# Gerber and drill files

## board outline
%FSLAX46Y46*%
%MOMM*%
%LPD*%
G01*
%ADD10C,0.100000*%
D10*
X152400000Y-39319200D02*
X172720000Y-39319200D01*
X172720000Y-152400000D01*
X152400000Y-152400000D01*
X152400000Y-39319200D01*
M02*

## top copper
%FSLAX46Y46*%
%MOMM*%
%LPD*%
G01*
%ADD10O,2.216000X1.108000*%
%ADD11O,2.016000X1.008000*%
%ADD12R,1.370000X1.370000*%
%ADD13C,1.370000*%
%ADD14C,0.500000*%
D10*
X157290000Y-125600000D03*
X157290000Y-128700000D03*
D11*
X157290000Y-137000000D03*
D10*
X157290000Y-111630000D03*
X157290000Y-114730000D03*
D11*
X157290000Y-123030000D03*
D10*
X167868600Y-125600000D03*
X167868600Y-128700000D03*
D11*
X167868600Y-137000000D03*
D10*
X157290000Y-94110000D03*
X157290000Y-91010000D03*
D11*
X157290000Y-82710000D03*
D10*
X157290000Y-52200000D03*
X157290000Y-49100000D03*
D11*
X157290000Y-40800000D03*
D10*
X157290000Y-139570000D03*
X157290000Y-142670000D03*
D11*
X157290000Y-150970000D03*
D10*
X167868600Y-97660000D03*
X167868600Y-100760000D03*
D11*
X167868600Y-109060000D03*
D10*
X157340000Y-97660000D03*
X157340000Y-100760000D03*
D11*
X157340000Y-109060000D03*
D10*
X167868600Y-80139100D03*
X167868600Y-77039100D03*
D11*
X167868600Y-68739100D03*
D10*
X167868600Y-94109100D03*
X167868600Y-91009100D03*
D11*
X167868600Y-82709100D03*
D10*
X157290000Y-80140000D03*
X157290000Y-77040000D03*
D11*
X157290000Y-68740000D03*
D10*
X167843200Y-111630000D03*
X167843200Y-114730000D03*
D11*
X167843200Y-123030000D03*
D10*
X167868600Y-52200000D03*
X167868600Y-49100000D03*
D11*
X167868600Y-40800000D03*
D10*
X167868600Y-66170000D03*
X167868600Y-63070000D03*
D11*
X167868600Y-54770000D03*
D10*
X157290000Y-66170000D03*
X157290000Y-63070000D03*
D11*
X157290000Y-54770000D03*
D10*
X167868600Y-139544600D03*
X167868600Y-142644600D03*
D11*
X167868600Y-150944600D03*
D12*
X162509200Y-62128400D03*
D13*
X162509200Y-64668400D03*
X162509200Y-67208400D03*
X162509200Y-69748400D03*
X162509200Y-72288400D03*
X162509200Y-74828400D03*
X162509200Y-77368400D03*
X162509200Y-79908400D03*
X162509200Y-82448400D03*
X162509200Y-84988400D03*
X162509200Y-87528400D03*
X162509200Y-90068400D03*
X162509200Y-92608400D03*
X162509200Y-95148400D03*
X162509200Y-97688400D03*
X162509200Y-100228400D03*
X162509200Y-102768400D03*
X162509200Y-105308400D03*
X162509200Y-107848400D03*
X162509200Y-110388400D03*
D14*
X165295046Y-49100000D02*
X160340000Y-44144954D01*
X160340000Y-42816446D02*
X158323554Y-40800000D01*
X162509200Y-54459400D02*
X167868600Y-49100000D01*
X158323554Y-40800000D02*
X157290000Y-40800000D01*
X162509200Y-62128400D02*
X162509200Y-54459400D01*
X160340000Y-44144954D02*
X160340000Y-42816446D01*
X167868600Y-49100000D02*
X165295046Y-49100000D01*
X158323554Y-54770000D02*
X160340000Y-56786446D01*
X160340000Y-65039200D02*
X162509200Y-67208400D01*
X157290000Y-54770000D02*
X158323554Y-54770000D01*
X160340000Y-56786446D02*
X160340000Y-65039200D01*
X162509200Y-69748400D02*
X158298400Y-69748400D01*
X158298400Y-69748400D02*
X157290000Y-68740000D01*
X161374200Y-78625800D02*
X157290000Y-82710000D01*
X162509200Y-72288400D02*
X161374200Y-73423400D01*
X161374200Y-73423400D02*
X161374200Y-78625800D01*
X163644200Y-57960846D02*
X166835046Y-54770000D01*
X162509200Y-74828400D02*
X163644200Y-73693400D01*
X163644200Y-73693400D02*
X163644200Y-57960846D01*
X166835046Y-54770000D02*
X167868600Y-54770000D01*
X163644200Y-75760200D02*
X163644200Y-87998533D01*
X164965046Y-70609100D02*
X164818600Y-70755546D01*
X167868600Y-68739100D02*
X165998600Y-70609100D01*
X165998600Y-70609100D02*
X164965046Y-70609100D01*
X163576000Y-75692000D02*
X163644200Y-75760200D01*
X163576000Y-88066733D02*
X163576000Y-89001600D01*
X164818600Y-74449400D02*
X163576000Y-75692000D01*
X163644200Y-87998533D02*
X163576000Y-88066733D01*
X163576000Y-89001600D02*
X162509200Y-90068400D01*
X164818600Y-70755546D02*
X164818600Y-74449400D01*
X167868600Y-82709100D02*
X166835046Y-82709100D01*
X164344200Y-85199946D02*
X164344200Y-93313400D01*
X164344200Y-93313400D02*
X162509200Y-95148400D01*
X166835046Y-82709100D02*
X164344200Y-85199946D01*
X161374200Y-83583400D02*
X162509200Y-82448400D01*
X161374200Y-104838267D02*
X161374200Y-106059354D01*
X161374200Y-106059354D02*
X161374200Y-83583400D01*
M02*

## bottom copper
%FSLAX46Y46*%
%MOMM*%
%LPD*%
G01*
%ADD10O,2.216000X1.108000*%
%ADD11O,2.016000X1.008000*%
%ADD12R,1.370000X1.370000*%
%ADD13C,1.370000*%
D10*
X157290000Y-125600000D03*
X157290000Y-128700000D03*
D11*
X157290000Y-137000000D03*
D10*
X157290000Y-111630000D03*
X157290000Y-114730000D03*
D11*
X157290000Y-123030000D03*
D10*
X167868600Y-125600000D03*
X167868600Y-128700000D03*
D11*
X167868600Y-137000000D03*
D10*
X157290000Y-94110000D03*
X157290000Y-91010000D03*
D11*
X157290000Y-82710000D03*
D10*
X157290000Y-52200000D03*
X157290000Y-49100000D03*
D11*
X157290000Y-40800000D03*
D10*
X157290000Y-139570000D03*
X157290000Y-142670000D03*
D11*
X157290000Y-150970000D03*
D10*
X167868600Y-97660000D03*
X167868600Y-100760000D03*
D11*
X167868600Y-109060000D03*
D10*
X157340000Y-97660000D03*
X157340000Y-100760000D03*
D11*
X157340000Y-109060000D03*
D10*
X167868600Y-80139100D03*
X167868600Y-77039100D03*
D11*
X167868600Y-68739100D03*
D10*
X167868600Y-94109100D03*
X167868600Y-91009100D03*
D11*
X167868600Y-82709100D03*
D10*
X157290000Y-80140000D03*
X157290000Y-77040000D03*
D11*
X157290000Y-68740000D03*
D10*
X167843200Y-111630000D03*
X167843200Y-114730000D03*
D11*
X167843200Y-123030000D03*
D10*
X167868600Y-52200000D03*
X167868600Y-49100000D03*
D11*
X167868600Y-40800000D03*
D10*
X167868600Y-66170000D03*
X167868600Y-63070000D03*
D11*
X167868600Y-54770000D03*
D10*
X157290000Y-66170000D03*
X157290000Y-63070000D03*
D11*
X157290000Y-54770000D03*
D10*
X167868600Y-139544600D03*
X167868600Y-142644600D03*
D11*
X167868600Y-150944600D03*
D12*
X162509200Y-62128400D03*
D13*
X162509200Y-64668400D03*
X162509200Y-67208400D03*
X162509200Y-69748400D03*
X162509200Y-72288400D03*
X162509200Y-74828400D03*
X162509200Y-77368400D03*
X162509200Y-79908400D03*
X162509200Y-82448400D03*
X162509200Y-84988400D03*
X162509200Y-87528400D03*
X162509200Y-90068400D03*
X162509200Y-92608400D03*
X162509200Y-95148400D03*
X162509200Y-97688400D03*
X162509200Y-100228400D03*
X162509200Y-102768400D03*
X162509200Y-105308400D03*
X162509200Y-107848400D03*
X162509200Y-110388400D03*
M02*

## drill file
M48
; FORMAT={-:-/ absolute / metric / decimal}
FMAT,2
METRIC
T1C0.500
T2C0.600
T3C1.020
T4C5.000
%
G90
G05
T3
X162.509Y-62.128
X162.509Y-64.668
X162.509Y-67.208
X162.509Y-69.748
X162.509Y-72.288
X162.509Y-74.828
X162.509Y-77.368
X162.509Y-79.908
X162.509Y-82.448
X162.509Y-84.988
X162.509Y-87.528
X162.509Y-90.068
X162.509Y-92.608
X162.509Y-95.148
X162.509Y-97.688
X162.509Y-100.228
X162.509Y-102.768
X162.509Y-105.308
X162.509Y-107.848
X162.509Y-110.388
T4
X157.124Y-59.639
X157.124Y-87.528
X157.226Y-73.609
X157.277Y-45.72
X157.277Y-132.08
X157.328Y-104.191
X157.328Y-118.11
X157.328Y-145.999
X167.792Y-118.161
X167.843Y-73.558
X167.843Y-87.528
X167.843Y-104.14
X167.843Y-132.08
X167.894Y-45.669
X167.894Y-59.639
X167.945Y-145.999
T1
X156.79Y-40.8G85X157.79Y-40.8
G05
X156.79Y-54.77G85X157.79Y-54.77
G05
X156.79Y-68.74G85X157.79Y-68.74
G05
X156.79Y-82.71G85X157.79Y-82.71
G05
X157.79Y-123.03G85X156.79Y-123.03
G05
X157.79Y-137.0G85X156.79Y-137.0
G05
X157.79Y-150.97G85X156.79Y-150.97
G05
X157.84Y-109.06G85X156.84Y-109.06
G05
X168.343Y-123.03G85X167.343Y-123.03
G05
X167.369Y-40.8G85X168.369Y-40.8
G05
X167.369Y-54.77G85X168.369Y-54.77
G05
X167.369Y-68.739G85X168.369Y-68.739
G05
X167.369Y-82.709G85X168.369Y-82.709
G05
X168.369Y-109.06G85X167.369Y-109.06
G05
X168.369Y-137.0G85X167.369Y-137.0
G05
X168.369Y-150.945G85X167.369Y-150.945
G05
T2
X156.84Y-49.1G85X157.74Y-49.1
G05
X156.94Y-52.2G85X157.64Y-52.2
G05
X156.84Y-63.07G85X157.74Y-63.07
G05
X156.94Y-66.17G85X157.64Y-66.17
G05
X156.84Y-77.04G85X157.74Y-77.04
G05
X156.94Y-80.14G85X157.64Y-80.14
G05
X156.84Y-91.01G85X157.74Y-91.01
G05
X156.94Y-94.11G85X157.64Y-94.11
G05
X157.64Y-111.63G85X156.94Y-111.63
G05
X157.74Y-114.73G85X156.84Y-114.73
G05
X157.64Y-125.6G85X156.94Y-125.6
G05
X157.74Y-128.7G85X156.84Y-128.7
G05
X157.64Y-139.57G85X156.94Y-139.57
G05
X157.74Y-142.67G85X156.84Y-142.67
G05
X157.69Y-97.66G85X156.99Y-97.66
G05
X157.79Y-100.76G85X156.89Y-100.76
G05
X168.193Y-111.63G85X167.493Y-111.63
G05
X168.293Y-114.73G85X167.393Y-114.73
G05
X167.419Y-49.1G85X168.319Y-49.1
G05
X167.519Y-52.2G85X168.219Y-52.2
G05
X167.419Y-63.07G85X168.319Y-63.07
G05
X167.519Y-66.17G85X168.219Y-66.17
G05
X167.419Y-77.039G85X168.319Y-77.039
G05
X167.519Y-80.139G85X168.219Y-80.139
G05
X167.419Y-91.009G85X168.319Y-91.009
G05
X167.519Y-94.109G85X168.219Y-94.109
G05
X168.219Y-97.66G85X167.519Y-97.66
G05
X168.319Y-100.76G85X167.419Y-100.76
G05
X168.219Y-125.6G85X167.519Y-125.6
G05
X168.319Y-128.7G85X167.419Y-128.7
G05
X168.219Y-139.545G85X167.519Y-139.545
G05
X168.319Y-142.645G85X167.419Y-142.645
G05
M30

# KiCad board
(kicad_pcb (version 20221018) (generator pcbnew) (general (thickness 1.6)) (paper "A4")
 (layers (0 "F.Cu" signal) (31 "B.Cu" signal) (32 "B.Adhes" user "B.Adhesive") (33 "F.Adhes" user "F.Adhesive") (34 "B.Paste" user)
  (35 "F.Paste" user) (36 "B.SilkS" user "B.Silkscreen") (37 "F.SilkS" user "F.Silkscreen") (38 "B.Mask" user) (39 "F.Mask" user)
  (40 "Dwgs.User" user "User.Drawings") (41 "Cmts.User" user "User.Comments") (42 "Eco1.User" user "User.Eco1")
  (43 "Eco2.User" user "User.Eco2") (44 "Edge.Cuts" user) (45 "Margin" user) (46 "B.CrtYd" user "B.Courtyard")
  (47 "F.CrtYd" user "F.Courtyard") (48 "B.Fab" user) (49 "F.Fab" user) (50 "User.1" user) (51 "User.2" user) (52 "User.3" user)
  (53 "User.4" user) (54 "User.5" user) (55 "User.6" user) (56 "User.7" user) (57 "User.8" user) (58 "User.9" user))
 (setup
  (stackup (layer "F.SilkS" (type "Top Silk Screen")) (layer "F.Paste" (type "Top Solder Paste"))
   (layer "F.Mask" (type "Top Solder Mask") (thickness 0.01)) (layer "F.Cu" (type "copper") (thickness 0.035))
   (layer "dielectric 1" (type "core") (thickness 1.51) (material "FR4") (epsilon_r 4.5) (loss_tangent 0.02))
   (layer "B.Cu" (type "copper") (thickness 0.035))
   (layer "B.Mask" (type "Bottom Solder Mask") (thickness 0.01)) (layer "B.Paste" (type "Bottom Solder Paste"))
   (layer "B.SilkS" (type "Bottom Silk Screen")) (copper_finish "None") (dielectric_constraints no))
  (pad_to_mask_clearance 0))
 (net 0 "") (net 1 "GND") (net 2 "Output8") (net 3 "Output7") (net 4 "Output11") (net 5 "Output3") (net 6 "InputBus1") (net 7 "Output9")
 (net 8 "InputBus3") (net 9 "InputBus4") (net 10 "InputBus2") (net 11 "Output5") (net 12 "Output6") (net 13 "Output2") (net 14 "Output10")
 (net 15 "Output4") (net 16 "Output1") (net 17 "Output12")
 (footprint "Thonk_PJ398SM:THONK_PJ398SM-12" (layer "F.Cu") (at 157.29 132.08 180)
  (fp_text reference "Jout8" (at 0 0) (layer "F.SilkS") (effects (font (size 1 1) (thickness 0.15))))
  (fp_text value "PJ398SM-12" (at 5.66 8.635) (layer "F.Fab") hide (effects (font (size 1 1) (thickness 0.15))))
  (pad "1" thru_hole oval (at 0 6.48 180) (size 2.216 1.108) (drill oval 1.3 0.6) (layers "*.Cu" "*.Mask") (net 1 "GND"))
  (pad "2" thru_hole oval (at 0 3.38 180) (size 2.216 1.108) (drill oval 1.5 0.6) (layers "*.Cu" "*.Mask") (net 1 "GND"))
  (pad "3" thru_hole oval (at 0 -4.92 180) (size 2.016 1.008) (drill oval 1.5 0.5) (layers "*.Cu" "*.Mask") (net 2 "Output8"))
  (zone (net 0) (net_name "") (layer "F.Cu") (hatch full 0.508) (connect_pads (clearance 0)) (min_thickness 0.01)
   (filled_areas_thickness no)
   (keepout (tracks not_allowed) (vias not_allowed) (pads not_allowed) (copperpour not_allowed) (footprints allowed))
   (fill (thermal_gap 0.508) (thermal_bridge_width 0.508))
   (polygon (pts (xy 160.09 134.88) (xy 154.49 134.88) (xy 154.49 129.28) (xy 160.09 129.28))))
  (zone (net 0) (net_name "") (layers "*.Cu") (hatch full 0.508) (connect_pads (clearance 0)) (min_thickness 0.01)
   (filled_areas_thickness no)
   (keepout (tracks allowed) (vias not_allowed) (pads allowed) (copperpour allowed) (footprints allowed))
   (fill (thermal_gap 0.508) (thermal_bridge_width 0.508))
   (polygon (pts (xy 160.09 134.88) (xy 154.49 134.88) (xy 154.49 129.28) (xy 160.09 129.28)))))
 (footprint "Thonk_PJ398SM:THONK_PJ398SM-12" (layer "F.Cu") (at 157.29 118.11 180)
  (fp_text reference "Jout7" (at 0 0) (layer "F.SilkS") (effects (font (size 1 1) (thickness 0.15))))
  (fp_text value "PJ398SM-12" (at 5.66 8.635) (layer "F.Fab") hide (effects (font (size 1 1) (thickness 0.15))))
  (pad "1" thru_hole oval (at 0 6.48 180) (size 2.216 1.108) (drill oval 1.3 0.6) (layers "*.Cu" "*.Mask") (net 1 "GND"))
  (pad "2" thru_hole oval (at 0 3.38 180) (size 2.216 1.108) (drill oval 1.5 0.6) (layers "*.Cu" "*.Mask") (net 1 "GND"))
  (pad "3" thru_hole oval (at 0 -4.92 180) (size 2.016 1.008) (drill oval 1.5 0.5) (layers "*.Cu" "*.Mask") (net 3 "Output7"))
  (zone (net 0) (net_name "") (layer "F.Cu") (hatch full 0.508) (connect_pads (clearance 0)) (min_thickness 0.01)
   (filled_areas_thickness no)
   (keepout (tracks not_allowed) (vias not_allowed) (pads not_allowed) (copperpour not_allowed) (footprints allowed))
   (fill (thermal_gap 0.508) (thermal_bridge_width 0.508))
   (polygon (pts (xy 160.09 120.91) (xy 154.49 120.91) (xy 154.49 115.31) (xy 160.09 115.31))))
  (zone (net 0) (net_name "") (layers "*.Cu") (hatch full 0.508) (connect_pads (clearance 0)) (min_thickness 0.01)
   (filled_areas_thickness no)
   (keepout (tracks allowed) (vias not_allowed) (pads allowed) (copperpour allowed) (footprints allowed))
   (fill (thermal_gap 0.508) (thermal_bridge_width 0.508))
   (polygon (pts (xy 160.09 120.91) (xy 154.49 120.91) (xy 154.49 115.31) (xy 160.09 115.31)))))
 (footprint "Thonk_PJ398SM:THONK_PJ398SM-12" (layer "F.Cu") (at 167.8686 132.08 180)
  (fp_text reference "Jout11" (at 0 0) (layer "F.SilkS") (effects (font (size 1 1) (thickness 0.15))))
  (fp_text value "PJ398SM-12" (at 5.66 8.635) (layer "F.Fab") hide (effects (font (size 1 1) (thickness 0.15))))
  (pad "1" thru_hole oval (at 0 6.48 180) (size 2.216 1.108) (drill oval 1.3 0.6) (layers "*.Cu" "*.Mask") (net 1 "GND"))
  (pad "2" thru_hole oval (at 0 3.38 180) (size 2.216 1.108) (drill oval 1.5 0.6) (layers "*.Cu" "*.Mask") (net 1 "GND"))
  (pad "3" thru_hole oval (at 0 -4.92 180) (size 2.016 1.008) (drill oval 1.5 0.5) (layers "*.Cu" "*.Mask") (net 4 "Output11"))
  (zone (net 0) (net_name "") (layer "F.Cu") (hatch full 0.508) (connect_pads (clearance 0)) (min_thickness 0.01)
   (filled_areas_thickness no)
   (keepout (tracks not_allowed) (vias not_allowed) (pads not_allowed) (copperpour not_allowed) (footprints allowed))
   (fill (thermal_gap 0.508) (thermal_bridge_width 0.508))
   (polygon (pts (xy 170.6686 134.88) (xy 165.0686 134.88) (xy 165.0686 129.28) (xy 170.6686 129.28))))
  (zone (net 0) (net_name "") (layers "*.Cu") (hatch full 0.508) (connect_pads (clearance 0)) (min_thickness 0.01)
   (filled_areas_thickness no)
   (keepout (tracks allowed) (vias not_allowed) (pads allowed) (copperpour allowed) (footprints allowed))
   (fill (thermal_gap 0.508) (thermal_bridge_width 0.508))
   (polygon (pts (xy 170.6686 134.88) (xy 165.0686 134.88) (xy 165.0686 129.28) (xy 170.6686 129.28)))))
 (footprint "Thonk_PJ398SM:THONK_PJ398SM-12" (layer "F.Cu") (at 157.29 87.63)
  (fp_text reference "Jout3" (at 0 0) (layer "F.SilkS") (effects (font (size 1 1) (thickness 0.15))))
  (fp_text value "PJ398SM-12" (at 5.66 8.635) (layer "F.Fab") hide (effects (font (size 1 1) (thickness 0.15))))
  (pad "1" thru_hole oval (at 0 6.48) (size 2.216 1.108) (drill oval 1.3 0.6) (layers "*.Cu" "*.Mask") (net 1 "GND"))
  (pad "2" thru_hole oval (at 0 3.38) (size 2.216 1.108) (drill oval 1.5 0.6) (layers "*.Cu" "*.Mask") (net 1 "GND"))
  (pad "3" thru_hole oval (at 0 -4.92) (size 2.016 1.008) (drill oval 1.5 0.5) (layers "*.Cu" "*.Mask") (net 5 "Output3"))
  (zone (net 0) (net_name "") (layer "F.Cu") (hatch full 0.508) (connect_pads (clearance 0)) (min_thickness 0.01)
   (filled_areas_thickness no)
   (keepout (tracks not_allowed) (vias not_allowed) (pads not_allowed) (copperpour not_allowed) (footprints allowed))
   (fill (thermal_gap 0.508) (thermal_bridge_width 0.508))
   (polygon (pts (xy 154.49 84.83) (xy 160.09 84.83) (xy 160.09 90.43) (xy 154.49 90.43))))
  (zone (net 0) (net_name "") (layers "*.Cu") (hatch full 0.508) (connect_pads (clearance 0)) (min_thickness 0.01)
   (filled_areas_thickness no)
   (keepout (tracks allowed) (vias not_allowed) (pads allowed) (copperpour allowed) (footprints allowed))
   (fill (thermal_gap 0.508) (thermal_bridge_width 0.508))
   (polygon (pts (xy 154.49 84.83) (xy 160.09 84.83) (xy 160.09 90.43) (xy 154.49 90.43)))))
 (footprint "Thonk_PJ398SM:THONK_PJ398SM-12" (layer "F.Cu") (at 157.29 45.72)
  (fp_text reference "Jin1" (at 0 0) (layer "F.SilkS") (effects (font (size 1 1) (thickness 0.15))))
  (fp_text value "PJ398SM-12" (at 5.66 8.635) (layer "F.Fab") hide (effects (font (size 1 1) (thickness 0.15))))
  (pad "1" thru_hole oval (at 0 6.48) (size 2.216 1.108) (drill oval 1.3 0.6) (layers "*.Cu" "*.Mask") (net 1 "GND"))
  (pad "2" thru_hole oval (at 0 3.38) (size 2.216 1.108) (drill oval 1.5 0.6) (layers "*.Cu" "*.Mask") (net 1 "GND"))
  (pad "3" thru_hole oval (at 0 -4.92) (size 2.016 1.008) (drill oval 1.5 0.5) (layers "*.Cu" "*.Mask") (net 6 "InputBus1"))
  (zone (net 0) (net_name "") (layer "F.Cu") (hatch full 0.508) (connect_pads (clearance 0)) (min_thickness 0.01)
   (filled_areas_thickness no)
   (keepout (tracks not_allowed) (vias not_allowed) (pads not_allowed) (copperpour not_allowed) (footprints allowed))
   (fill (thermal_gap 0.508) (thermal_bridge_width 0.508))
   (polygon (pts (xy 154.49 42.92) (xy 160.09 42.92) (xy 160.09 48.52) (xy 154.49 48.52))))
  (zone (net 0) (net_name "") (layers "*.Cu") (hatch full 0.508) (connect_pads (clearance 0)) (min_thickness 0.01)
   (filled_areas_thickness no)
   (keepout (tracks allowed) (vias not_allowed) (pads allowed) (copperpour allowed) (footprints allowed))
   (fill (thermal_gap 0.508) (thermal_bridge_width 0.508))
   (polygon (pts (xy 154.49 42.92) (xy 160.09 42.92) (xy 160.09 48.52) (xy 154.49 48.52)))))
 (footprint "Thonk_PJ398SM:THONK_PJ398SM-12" (layer "F.Cu") (at 157.29 146.05 180)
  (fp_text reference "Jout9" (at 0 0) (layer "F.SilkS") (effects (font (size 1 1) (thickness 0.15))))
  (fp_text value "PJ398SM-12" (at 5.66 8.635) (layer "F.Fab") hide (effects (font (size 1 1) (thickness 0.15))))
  (pad "1" thru_hole oval (at 0 6.48 180) (size 2.216 1.108) (drill oval 1.3 0.6) (layers "*.Cu" "*.Mask") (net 1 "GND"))
  (pad "2" thru_hole oval (at 0 3.38 180) (size 2.216 1.108) (drill oval 1.5 0.6) (layers "*.Cu" "*.Mask") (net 1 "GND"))
  (pad "3" thru_hole oval (at 0 -4.92 180) (size 2.016 1.008) (drill oval 1.5 0.5) (layers "*.Cu" "*.Mask") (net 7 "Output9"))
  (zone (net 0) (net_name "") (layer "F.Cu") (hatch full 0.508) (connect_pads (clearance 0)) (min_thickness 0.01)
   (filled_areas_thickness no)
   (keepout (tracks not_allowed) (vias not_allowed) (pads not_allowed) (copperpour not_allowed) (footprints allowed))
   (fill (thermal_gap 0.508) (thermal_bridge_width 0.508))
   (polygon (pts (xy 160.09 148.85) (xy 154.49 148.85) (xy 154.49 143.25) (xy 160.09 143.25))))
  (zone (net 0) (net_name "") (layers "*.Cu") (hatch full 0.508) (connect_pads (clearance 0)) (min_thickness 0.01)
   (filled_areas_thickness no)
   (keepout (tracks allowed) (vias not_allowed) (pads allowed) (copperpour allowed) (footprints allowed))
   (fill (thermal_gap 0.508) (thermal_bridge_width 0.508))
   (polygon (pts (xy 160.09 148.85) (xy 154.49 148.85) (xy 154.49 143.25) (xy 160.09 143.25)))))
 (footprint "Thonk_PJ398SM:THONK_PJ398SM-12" (layer "F.Cu") (at 167.8686 104.14 180)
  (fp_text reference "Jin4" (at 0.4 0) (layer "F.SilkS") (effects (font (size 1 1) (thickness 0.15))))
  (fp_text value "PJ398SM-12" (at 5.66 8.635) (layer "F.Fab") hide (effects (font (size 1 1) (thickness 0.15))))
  (pad "1" thru_hole oval (at 0 6.48 180) (size 2.216 1.108) (drill oval 1.3 0.6) (layers "*.Cu" "*.Mask") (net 1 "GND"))
  (pad "2" thru_hole oval (at 0 3.38 180) (size 2.216 1.108) (drill oval 1.5 0.6) (layers "*.Cu" "*.Mask") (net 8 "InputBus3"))
  (pad "3" thru_hole oval (at 0 -4.92 180) (size 2.016 1.008) (drill oval 1.5 0.5) (layers "*.Cu" "*.Mask") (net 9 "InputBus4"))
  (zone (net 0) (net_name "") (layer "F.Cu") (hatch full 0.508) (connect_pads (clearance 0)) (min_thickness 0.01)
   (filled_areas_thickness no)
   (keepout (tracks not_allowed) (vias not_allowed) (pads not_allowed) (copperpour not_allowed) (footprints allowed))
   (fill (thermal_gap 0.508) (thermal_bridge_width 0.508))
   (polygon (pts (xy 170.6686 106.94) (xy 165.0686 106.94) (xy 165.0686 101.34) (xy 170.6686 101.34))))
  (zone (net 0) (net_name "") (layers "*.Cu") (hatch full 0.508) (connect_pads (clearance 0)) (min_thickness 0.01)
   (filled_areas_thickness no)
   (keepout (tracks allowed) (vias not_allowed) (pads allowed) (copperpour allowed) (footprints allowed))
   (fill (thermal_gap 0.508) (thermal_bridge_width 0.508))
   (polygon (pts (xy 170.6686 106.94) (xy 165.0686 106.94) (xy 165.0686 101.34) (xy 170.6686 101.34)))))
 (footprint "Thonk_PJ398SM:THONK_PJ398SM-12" (layer "F.Cu") (at 157.34 104.14 180)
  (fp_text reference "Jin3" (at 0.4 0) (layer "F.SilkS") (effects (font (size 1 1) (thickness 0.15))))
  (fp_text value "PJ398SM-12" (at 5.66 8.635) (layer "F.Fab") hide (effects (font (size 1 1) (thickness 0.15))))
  (pad "1" thru_hole oval (at 0 6.48 180) (size 2.216 1.108) (drill oval 1.3 0.6) (layers "*.Cu" "*.Mask") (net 1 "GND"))
  (pad "2" thru_hole oval (at 0 3.38 180) (size 2.216 1.108) (drill oval 1.5 0.6) (layers "*.Cu" "*.Mask") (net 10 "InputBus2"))
  (pad "3" thru_hole oval (at 0 -4.92 180) (size 2.016 1.008) (drill oval 1.5 0.5) (layers "*.Cu" "*.Mask") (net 8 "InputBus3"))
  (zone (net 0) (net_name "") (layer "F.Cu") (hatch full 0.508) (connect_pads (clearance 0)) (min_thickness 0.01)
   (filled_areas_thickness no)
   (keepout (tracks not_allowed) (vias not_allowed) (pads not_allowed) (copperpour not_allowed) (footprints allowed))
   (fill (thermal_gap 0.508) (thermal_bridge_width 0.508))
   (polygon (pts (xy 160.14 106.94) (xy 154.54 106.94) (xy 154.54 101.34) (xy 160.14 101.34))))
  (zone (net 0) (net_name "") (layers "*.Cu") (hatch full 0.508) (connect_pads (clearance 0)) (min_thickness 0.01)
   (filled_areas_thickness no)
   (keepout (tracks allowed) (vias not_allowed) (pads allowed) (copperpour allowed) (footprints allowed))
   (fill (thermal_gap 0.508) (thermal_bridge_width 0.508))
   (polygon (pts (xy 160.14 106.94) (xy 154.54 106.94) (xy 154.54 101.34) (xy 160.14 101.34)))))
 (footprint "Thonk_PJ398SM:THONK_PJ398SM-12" (layer "F.Cu") (at 167.8686 73.6591)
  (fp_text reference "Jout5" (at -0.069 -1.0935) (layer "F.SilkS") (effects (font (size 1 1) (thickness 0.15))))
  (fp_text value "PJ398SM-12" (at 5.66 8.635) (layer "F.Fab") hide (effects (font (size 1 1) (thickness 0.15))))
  (pad "1" thru_hole oval (at 0 6.48) (size 2.216 1.108) (drill oval 1.3 0.6) (layers "*.Cu" "*.Mask") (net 1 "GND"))
  (pad "2" thru_hole oval (at 0 3.38) (size 2.216 1.108) (drill oval 1.5 0.6) (layers "*.Cu" "*.Mask") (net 1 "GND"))
  (pad "3" thru_hole oval (at 0 -4.92) (size 2.016 1.008) (drill oval 1.5 0.5) (layers "*.Cu" "*.Mask") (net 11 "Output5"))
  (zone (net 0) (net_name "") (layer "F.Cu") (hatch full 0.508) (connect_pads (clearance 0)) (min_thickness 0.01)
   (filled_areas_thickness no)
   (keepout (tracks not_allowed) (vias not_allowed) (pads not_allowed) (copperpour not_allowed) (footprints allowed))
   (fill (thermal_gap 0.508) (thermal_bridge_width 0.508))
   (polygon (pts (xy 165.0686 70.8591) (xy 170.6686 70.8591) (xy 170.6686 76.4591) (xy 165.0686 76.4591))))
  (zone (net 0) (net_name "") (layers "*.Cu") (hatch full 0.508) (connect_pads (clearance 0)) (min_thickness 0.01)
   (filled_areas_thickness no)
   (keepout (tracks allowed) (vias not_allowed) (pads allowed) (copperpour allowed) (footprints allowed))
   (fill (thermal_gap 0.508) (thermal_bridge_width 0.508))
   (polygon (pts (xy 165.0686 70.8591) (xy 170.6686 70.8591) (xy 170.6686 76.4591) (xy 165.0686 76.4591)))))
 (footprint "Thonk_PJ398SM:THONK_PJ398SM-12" (layer "F.Cu") (at 167.8686 87.6291)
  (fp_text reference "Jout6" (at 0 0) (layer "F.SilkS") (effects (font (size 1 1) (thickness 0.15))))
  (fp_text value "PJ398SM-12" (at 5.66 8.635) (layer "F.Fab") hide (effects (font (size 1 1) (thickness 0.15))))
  (pad "1" thru_hole oval (at 0 6.48) (size 2.216 1.108) (drill oval 1.3 0.6) (layers "*.Cu" "*.Mask") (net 1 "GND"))
  (pad "2" thru_hole oval (at 0 3.38) (size 2.216 1.108) (drill oval 1.5 0.6) (layers "*.Cu" "*.Mask") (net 1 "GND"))
  (pad "3" thru_hole oval (at 0 -4.92) (size 2.016 1.008) (drill oval 1.5 0.5) (layers "*.Cu" "*.Mask") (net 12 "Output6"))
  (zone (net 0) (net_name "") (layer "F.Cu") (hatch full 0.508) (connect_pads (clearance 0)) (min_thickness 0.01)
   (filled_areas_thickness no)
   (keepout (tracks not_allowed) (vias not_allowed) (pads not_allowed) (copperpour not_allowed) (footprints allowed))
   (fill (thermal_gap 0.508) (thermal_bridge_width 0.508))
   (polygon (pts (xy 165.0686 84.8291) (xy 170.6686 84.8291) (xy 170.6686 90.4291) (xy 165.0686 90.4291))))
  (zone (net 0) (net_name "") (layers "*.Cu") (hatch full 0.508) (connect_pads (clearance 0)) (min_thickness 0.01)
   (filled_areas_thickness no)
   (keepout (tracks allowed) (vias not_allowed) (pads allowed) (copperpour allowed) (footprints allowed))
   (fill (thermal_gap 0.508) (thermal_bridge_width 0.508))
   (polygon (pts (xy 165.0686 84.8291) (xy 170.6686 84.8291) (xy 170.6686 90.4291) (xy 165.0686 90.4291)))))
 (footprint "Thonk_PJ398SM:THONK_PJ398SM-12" (layer "F.Cu") (at 157.29 73.66)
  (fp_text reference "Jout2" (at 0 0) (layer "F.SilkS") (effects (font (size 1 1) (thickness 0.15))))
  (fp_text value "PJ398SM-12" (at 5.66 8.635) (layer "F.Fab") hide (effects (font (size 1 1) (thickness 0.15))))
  (pad "1" thru_hole oval (at 0 6.48) (size 2.216 1.108) (drill oval 1.3 0.6) (layers "*.Cu" "*.Mask") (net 1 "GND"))
  (pad "2" thru_hole oval (at 0 3.38) (size 2.216 1.108) (drill oval 1.5 0.6) (layers "*.Cu" "*.Mask") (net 1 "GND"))
  (pad "3" thru_hole oval (at 0 -4.92) (size 2.016 1.008) (drill oval 1.5 0.5) (layers "*.Cu" "*.Mask") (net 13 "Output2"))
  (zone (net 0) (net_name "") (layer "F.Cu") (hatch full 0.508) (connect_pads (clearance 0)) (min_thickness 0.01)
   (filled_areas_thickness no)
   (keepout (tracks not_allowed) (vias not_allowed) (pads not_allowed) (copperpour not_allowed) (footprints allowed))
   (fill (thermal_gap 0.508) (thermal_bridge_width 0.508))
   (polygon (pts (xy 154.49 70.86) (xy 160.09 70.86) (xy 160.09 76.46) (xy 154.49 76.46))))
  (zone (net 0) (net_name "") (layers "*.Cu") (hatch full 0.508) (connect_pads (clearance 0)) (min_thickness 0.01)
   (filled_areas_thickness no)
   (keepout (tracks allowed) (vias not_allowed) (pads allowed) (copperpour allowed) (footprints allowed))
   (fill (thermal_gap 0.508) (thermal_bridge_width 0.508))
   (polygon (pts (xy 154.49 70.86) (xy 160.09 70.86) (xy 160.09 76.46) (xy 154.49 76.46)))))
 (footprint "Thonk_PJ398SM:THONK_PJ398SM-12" (layer "F.Cu") (at 167.8432 118.11 180)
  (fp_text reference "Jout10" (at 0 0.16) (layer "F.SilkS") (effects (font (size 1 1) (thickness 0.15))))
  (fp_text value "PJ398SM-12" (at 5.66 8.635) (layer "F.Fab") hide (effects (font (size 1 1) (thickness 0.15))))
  (pad "1" thru_hole oval (at 0 6.48 180) (size 2.216 1.108) (drill oval 1.3 0.6) (layers "*.Cu" "*.Mask") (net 1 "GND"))
  (pad "2" thru_hole oval (at 0 3.38 180) (size 2.216 1.108) (drill oval 1.5 0.6) (layers "*.Cu" "*.Mask") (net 1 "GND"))
  (pad "3" thru_hole oval (at 0 -4.92 180) (size 2.016 1.008) (drill oval 1.5 0.5) (layers "*.Cu" "*.Mask") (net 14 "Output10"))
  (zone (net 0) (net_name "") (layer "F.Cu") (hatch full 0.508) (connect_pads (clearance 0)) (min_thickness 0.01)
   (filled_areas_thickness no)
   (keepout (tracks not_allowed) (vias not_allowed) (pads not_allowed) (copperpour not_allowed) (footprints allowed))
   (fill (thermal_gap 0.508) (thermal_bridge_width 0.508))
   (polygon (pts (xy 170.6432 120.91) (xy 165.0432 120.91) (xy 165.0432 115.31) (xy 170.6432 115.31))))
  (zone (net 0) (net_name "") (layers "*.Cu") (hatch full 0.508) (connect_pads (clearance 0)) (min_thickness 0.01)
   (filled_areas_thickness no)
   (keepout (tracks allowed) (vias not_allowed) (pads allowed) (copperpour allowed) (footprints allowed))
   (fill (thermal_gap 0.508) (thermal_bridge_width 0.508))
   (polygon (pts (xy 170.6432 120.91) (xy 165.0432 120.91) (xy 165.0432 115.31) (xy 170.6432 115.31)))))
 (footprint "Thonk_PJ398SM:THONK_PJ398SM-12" (layer "F.Cu") (at 167.8686 45.72)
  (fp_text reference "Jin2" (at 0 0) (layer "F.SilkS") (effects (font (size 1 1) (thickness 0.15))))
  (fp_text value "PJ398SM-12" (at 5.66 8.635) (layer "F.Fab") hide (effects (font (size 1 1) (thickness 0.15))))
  (pad "1" thru_hole oval (at 0 6.48) (size 2.216 1.108) (drill oval 1.3 0.6) (layers "*.Cu" "*.Mask") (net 1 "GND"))
  (pad "2" thru_hole oval (at 0 3.38) (size 2.216 1.108) (drill oval 1.5 0.6) (layers "*.Cu" "*.Mask") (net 6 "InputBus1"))
  (pad "3" thru_hole oval (at 0 -4.92) (size 2.016 1.008) (drill oval 1.5 0.5) (layers "*.Cu" "*.Mask") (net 10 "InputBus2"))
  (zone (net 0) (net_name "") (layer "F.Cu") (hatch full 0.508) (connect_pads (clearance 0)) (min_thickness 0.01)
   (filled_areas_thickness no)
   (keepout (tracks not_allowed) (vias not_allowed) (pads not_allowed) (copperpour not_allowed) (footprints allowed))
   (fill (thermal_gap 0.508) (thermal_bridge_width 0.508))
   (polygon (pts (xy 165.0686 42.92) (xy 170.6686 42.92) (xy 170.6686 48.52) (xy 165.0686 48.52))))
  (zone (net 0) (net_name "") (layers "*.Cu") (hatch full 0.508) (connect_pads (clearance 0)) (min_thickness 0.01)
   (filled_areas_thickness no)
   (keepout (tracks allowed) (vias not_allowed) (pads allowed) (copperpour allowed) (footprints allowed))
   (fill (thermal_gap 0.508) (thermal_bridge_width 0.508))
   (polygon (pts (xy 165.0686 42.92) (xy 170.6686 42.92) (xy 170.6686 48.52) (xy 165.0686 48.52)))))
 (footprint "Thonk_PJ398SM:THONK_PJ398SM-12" (layer "F.Cu") (at 167.8686 59.69)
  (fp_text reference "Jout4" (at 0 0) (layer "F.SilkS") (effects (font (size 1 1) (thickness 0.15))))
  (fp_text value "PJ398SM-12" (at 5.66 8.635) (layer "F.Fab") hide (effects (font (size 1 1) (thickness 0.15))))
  (pad "1" thru_hole oval (at 0 6.48) (size 2.216 1.108) (drill oval 1.3 0.6) (layers "*.Cu" "*.Mask") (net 1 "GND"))
  (pad "2" thru_hole oval (at 0 3.38) (size 2.216 1.108) (drill oval 1.5 0.6) (layers "*.Cu" "*.Mask") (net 1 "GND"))
  (pad "3" thru_hole oval (at 0 -4.92) (size 2.016 1.008) (drill oval 1.5 0.5) (layers "*.Cu" "*.Mask") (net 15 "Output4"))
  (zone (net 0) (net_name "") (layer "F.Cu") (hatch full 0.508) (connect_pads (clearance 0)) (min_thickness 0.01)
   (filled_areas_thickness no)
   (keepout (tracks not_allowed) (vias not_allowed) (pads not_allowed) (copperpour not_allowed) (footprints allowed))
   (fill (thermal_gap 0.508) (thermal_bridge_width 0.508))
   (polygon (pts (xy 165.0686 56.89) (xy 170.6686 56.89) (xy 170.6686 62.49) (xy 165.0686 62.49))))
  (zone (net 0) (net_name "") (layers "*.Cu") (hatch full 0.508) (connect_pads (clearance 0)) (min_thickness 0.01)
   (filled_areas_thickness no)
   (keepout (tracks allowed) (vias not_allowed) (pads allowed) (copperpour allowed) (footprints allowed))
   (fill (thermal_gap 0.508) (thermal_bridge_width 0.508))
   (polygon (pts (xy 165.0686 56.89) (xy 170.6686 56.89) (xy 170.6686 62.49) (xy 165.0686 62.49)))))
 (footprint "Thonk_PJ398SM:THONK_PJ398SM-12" (layer "F.Cu") (at 157.29 59.69)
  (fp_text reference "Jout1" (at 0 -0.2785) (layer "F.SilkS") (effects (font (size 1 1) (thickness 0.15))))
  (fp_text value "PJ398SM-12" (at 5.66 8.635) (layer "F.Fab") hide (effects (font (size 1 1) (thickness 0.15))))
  (pad "1" thru_hole oval (at 0 6.48) (size 2.216 1.108) (drill oval 1.3 0.6) (layers "*.Cu" "*.Mask") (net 1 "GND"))
  (pad "2" thru_hole oval (at 0 3.38) (size 2.216 1.108) (drill oval 1.5 0.6) (layers "*.Cu" "*.Mask") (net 1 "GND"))
  (pad "3" thru_hole oval (at 0 -4.92) (size 2.016 1.008) (drill oval 1.5 0.5) (layers "*.Cu" "*.Mask") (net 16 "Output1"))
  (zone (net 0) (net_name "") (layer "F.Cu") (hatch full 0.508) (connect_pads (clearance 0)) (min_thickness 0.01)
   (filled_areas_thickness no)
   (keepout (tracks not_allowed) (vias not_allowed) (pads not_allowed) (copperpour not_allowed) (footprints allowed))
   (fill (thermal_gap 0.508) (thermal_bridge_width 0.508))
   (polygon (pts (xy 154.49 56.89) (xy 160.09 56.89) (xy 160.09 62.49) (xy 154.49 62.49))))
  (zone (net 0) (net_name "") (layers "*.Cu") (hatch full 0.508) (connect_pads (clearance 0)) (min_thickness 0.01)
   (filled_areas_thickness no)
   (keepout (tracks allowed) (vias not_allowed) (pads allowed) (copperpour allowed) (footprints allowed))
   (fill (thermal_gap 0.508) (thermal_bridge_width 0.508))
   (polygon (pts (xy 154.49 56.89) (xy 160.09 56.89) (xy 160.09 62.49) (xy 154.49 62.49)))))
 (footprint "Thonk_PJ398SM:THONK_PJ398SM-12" (layer "F.Cu") (at 167.8686 146.0246 180)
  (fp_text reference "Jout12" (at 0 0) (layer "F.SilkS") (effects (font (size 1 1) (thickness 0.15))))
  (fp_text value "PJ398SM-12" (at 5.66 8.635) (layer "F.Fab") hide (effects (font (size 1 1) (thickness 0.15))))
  (pad "1" thru_hole oval (at 0 6.48 180) (size 2.216 1.108) (drill oval 1.3 0.6) (layers "*.Cu" "*.Mask") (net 1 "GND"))
  (pad "2" thru_hole oval (at 0 3.38 180) (size 2.216 1.108) (drill oval 1.5 0.6) (layers "*.Cu" "*.Mask") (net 1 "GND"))
  (pad "3" thru_hole oval (at 0 -4.92 180) (size 2.016 1.008) (drill oval 1.5 0.5) (layers "*.Cu" "*.Mask") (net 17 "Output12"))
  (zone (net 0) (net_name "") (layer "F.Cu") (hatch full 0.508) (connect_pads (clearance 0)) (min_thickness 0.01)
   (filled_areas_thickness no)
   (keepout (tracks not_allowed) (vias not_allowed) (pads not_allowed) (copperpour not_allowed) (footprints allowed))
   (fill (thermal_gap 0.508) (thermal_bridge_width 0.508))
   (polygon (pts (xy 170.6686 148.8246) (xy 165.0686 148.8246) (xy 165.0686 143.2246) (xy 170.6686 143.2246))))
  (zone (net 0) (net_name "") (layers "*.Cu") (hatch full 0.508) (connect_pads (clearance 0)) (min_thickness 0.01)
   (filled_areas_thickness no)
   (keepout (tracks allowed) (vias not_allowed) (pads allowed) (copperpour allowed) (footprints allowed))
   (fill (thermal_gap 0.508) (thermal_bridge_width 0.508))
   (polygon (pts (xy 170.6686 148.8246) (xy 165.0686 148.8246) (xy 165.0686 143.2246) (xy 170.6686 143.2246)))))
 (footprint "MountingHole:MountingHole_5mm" (layer "B.Cu") (at 167.7924 118.1608 180)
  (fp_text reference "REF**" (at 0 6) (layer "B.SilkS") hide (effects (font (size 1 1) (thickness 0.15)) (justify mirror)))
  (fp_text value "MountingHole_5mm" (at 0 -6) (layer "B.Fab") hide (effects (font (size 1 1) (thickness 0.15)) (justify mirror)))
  (pad "" np_thru_hole circle (at 0 0 180) (size 5 5) (drill 5) (layers "F&B.Cu" "*.Mask")))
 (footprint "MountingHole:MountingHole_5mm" (layer "B.Cu") (at 157.3276 104.1908 180)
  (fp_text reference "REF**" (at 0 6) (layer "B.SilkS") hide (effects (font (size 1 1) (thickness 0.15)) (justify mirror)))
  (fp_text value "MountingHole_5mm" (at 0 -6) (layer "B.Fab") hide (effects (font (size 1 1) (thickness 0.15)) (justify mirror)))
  (pad "" np_thru_hole circle (at 0 0 180) (size 5 5) (drill 5) (layers "F&B.Cu" "*.Mask")))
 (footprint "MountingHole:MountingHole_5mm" (layer "B.Cu") (at 167.894 45.6692 180)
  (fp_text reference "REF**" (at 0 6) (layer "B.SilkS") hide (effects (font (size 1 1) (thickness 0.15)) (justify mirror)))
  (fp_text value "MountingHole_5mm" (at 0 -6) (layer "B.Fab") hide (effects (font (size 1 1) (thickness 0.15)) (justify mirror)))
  (pad "" np_thru_hole circle (at 0 0 180) (size 5 5) (drill 5) (layers "F&B.Cu" "*.Mask")))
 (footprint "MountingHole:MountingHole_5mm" (layer "B.Cu") (at 157.3276 118.11 180)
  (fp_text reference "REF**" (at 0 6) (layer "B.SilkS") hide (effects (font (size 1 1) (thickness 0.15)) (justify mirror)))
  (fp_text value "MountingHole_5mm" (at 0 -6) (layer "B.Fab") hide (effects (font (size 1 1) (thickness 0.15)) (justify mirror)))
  (pad "" np_thru_hole circle (at 0 0 180) (size 5 5) (drill 5) (layers "F&B.Cu" "*.Mask")))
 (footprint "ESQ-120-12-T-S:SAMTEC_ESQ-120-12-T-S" (layer "B.Cu") (at 162.5092 62.1284 -90)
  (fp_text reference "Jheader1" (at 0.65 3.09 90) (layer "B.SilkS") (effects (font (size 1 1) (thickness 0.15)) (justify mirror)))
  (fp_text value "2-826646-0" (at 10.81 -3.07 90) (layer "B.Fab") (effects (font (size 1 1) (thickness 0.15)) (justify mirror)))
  (pad "01" thru_hole rect (at 0 0 270) (size 1.37 1.37) (drill 1.02) (layers "*.Cu" "*.Mask") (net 6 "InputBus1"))
  (pad "02" thru_hole circle (at 2.54 0 270) (size 1.37 1.37) (drill 1.02) (layers "*.Cu" "*.Mask") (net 10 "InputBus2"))
  (pad "03" thru_hole circle (at 5.08 0 270) (size 1.37 1.37) (drill 1.02) (layers "*.Cu" "*.Mask") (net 16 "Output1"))
  (pad "04" thru_hole circle (at 7.62 0 270) (size 1.37 1.37) (drill 1.02) (layers "*.Cu" "*.Mask") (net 13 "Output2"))
  (pad "05" thru_hole circle (at 10.16 0 270) (size 1.37 1.37) (drill 1.02) (layers "*.Cu" "*.Mask") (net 5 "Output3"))
  (pad "06" thru_hole circle (at 12.7 0 270) (size 1.37 1.37) (drill 1.02) (layers "*.Cu" "*.Mask") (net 15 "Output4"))
  (pad "07" thru_hole circle (at 15.24 0 270) (size 1.37 1.37) (drill 1.02) (layers "*.Cu" "*.Mask") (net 7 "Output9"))
  (pad "08" thru_hole circle (at 17.78 0 270) (size 1.37 1.37) (drill 1.02) (layers "*.Cu" "*.Mask") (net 14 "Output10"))
  (pad "09" thru_hole circle (at 20.32 0 270) (size 1.37 1.37) (drill 1.02) (layers "*.Cu" "*.Mask") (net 8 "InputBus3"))
  (pad "10" thru_hole circle (at 22.86 0 270) (size 1.37 1.37) (drill 1.02) (layers "*.Cu" "*.Mask") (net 9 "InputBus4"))
  (pad "11" thru_hole circle (at 25.4 0 270) (size 1.37 1.37) (drill 1.02) (layers "*.Cu" "*.Mask") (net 3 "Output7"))
  (pad "12" thru_hole circle (at 27.94 0 270) (size 1.37 1.37) (drill 1.02) (layers "*.Cu" "*.Mask") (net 11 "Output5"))
  (pad "13" thru_hole circle (at 30.48 0 270) (size 1.37 1.37) (drill 1.02) (layers "*.Cu" "*.Mask") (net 2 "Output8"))
  (pad "14" thru_hole circle (at 33.02 0 270) (size 1.37 1.37) (drill 1.02) (layers "*.Cu" "*.Mask") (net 12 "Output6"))
  (pad "15" thru_hole circle (at 35.56 0 270) (size 1.37 1.37) (drill 1.02) (layers "*.Cu" "*.Mask") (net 4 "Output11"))
  (pad "16" thru_hole circle (at 38.1 0 270) (size 1.37 1.37) (drill 1.02) (layers "*.Cu" "*.Mask") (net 17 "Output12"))
  (pad "17" thru_hole circle (at 40.64 0 270) (size 1.37 1.37) (drill 1.02) (layers "*.Cu" "*.Mask") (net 1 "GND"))
  (pad "18" thru_hole circle (at 43.18 0 270) (size 1.37 1.37) (drill 1.02) (layers "*.Cu" "*.Mask") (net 1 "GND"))
  (pad "19" thru_hole circle (at 45.72 0 270) (size 1.37 1.37) (drill 1.02) (layers "*.Cu" "*.Mask") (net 1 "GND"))
  (pad "20" thru_hole circle (at 48.26 0 270) (size 1.37 1.37) (drill 1.02) (layers "*.Cu" "*.Mask") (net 1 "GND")))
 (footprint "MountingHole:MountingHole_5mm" (layer "B.Cu") (at 167.8432 73.5584 180)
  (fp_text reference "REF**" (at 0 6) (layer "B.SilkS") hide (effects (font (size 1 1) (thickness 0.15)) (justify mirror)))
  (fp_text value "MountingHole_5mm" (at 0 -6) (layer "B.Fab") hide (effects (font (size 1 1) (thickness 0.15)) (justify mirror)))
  (pad "" np_thru_hole circle (at 0 0 180) (size 5 5) (drill 5) (layers "F&B.Cu" "*.Mask")))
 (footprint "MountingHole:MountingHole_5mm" (layer "B.Cu") (at 157.2768 45.72 180)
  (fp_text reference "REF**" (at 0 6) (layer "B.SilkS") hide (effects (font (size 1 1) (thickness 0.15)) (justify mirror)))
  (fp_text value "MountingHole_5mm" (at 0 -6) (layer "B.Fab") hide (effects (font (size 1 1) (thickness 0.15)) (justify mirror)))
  (pad "" np_thru_hole circle (at 0 0 180) (size 5 5) (drill 5) (layers "*.Cu" "*.Mask")))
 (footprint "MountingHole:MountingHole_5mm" (layer "B.Cu") (at 167.8432 132.08 180)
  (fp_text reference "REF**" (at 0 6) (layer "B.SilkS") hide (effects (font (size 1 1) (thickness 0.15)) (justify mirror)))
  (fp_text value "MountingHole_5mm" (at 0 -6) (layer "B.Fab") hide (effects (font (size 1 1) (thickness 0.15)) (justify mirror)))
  (pad "" np_thru_hole circle (at 0 0 180) (size 5 5) (drill 5) (layers "F&B.Cu" "*.Mask")))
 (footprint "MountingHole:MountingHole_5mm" (layer "B.Cu") (at 167.894 59.6392 180)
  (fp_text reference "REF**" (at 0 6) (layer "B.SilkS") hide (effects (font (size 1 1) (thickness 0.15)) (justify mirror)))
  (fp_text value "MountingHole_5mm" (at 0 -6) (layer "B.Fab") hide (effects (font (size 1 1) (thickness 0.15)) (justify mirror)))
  (pad "" np_thru_hole circle (at 0 0 180) (size 5 5) (drill 5) (layers "F&B.Cu" "*.Mask")))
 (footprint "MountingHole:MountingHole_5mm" (layer "B.Cu") (at 157.1244 59.6392 180)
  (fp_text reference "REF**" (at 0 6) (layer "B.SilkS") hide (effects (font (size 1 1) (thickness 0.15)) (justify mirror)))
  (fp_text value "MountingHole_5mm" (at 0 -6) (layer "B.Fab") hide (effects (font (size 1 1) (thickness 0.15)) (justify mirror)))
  (pad "" np_thru_hole circle (at 0 0 180) (size 5 5) (drill 5) (layers "F&B.Cu" "*.Mask")))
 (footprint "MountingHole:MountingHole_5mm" (layer "B.Cu") (at 157.3276 145.9992 180)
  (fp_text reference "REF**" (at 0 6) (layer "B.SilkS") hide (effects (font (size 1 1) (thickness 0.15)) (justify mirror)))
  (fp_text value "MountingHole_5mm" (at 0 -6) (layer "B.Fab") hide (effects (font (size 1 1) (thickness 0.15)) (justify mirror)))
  (pad "" np_thru_hole circle (at 0 0 180) (size 5 5) (drill 5) (layers "F&B.Cu" "*.Mask")))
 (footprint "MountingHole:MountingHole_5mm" (layer "B.Cu") (at 157.1244 87.5284 180)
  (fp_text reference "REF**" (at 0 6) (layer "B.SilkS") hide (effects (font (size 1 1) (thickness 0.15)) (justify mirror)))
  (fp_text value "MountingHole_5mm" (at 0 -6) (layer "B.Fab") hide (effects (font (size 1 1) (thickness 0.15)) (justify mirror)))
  (pad "" np_thru_hole circle (at 0 0 180) (size 5 5) (drill 5) (layers "F&B.Cu" "*.Mask")))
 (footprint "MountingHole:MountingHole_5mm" (layer "B.Cu") (at 157.2768 132.08 180)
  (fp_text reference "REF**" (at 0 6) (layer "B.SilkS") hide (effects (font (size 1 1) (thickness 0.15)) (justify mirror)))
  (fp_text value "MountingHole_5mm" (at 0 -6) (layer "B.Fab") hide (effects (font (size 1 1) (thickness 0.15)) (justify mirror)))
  (pad "" np_thru_hole circle (at 0 0 180) (size 5 5) (drill 5) (layers "F&B.Cu" "*.Mask")))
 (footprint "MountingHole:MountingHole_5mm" (layer "B.Cu") (at 167.8432 87.5284 180)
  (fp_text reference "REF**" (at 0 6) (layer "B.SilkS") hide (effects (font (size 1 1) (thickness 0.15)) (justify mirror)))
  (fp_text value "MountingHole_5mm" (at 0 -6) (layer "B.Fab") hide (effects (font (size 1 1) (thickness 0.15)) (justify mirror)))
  (pad "" np_thru_hole circle (at 0 0 180) (size 5 5) (drill 5) (layers "F&B.Cu" "*.Mask")))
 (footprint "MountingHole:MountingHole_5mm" (layer "B.Cu") (at 167.8432 104.14 180)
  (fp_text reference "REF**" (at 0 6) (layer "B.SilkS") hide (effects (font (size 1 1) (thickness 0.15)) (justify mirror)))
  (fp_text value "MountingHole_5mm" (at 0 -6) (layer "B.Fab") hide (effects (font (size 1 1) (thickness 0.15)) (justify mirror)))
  (pad "" np_thru_hole circle (at 0 0 180) (size 5 5) (drill 5) (layers "F&B.Cu" "*.Mask")))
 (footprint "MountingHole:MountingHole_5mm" (layer "B.Cu") (at 157.226 73.6092 180)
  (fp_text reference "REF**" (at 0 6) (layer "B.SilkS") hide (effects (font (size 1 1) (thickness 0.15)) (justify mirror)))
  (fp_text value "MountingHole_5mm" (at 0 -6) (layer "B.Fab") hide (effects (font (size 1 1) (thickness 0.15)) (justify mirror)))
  (pad "" np_thru_hole circle (at 0 0 180) (size 5 5) (drill 5) (layers "F&B.Cu" "*.Mask")))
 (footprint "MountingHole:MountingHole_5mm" (layer "B.Cu") (at 167.9448 145.9992 180)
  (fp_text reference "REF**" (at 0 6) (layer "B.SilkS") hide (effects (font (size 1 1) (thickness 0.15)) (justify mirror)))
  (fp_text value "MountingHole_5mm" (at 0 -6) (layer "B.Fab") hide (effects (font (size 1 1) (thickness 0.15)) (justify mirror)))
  (pad "" np_thru_hole circle (at 0 0 180) (size 5 5) (drill 5) (layers "F&B.Cu" "*.Mask")))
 (gr_rect (start 152.4 39.3192) (end 172.72 152.4) (stroke (width 0.1) (type solid)) (fill none) (layer "Edge.Cuts"))
 (segment (start 165.295046 49.1) (end 160.34 44.144954) (width 0.5) (layer "F.Cu") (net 6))
 (segment (start 160.34 42.816446) (end 158.323554 40.8) (width 0.5) (layer "F.Cu") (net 6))
 (segment (start 162.5092 54.4594) (end 167.8686 49.1) (width 0.5) (layer "F.Cu") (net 6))
 (segment (start 158.323554 40.8) (end 157.29 40.8) (width 0.5) (layer "F.Cu") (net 6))
 (segment (start 162.5092 62.1284) (end 162.5092 54.4594) (width 0.5) (layer "F.Cu") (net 6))
 (segment (start 160.34 44.144954) (end 160.34 42.816446) (width 0.5) (layer "F.Cu") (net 6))
 (segment (start 167.8686 49.1) (end 165.295046 49.1) (width 0.5) (layer "F.Cu") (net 6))
 (segment (start 158.323554 54.77) (end 160.34 56.786446) (width 0.5) (layer "F.Cu") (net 16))
 (segment (start 160.34 65.0392) (end 162.5092 67.2084) (width 0.5) (layer "F.Cu") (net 16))
 (segment (start 157.29 54.77) (end 158.323554 54.77) (width 0.5) (layer "F.Cu") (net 16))
 (segment (start 160.34 56.786446) (end 160.34 65.0392) (width 0.5) (layer "F.Cu") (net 16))
 (segment (start 162.5092 69.7484) (end 158.2984 69.7484) (width 0.5) (layer "F.Cu") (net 13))
 (segment (start 158.2984 69.7484) (end 157.29 68.74) (width 0.5) (layer "F.Cu") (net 13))
 (segment (start 161.3742 78.6258) (end 157.29 82.71) (width 0.5) (layer "F.Cu") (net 5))
 (segment (start 162.5092 72.2884) (end 161.3742 73.4234) (width 0.5) (layer "F.Cu") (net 5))
 (segment (start 161.3742 73.4234) (end 161.3742 78.6258) (width 0.5) (layer "F.Cu") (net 5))
 (segment (start 163.6442 57.960846) (end 166.835046 54.77) (width 0.5) (layer "F.Cu") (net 15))
 (segment (start 162.5092 74.8284) (end 163.6442 73.6934) (width 0.5) (layer "F.Cu") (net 15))
 (segment (start 163.6442 73.6934) (end 163.6442 57.960846) (width 0.5) (layer "F.Cu") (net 15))
 (segment (start 166.835046 54.77) (end 167.8686 54.77) (width 0.5) (layer "F.Cu") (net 15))
 (segment (start 163.6442 75.7602) (end 163.6442 87.998533) (width 0.5) (layer "F.Cu") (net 11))
 (segment (start 164.965046 70.6091) (end 164.8186 70.755546) (width 0.5) (layer "F.Cu") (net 11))
 (segment (start 167.8686 68.7391) (end 165.9986 70.6091) (width 0.5) (layer "F.Cu") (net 11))
 (segment (start 165.9986 70.6091) (end 164.965046 70.6091) (width 0.5) (layer "F.Cu") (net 11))
 (segment (start 163.576 75.692) (end 163.6442 75.7602) (width 0.5) (layer "F.Cu") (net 11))
 (segment (start 163.576 88.066733) (end 163.576 89.0016) (width 0.5) (layer "F.Cu") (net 11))
 (segment (start 164.8186 74.4494) (end 163.576 75.692) (width 0.5) (layer "F.Cu") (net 11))
 (segment (start 163.6442 87.998533) (end 163.576 88.066733) (width 0.5) (layer "F.Cu") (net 11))
 (segment (start 163.576 89.0016) (end 162.5092 90.0684) (width 0.5) (layer "F.Cu") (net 11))
 (segment (start 164.8186 70.755546) (end 164.8186 74.4494) (width 0.5) (layer "F.Cu") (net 11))
 (segment (start 167.8686 82.7091) (end 166.835046 82.7091) (width 0.5) (layer "F.Cu") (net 12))
 (segment (start 164.3442 85.199946) (end 164.3442 93.3134) (width 0.5) (layer "F.Cu") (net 12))
 (segment (start 164.3442 93.3134) (end 162.5092 95.1484) (width 0.5) (layer "F.Cu") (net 12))
 (segment (start 166.835046 82.7091) (end 164.3442 85.199946) (width 0.5) (layer "F.Cu") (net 12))
 (segment (start 161.3742 83.5834) (end 162.5092 82.4484) (width 0.5) (layer "F.Cu") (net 8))
 (segment (start 161.3742 104.838267) (end 161.3742 106.059354) (width 0.5) (layer "F.Cu") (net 8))
 (segment (start 161.3742 106.059354) (end 161.3742 83.5834) (width 0.5) (layer "F.Cu") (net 8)))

